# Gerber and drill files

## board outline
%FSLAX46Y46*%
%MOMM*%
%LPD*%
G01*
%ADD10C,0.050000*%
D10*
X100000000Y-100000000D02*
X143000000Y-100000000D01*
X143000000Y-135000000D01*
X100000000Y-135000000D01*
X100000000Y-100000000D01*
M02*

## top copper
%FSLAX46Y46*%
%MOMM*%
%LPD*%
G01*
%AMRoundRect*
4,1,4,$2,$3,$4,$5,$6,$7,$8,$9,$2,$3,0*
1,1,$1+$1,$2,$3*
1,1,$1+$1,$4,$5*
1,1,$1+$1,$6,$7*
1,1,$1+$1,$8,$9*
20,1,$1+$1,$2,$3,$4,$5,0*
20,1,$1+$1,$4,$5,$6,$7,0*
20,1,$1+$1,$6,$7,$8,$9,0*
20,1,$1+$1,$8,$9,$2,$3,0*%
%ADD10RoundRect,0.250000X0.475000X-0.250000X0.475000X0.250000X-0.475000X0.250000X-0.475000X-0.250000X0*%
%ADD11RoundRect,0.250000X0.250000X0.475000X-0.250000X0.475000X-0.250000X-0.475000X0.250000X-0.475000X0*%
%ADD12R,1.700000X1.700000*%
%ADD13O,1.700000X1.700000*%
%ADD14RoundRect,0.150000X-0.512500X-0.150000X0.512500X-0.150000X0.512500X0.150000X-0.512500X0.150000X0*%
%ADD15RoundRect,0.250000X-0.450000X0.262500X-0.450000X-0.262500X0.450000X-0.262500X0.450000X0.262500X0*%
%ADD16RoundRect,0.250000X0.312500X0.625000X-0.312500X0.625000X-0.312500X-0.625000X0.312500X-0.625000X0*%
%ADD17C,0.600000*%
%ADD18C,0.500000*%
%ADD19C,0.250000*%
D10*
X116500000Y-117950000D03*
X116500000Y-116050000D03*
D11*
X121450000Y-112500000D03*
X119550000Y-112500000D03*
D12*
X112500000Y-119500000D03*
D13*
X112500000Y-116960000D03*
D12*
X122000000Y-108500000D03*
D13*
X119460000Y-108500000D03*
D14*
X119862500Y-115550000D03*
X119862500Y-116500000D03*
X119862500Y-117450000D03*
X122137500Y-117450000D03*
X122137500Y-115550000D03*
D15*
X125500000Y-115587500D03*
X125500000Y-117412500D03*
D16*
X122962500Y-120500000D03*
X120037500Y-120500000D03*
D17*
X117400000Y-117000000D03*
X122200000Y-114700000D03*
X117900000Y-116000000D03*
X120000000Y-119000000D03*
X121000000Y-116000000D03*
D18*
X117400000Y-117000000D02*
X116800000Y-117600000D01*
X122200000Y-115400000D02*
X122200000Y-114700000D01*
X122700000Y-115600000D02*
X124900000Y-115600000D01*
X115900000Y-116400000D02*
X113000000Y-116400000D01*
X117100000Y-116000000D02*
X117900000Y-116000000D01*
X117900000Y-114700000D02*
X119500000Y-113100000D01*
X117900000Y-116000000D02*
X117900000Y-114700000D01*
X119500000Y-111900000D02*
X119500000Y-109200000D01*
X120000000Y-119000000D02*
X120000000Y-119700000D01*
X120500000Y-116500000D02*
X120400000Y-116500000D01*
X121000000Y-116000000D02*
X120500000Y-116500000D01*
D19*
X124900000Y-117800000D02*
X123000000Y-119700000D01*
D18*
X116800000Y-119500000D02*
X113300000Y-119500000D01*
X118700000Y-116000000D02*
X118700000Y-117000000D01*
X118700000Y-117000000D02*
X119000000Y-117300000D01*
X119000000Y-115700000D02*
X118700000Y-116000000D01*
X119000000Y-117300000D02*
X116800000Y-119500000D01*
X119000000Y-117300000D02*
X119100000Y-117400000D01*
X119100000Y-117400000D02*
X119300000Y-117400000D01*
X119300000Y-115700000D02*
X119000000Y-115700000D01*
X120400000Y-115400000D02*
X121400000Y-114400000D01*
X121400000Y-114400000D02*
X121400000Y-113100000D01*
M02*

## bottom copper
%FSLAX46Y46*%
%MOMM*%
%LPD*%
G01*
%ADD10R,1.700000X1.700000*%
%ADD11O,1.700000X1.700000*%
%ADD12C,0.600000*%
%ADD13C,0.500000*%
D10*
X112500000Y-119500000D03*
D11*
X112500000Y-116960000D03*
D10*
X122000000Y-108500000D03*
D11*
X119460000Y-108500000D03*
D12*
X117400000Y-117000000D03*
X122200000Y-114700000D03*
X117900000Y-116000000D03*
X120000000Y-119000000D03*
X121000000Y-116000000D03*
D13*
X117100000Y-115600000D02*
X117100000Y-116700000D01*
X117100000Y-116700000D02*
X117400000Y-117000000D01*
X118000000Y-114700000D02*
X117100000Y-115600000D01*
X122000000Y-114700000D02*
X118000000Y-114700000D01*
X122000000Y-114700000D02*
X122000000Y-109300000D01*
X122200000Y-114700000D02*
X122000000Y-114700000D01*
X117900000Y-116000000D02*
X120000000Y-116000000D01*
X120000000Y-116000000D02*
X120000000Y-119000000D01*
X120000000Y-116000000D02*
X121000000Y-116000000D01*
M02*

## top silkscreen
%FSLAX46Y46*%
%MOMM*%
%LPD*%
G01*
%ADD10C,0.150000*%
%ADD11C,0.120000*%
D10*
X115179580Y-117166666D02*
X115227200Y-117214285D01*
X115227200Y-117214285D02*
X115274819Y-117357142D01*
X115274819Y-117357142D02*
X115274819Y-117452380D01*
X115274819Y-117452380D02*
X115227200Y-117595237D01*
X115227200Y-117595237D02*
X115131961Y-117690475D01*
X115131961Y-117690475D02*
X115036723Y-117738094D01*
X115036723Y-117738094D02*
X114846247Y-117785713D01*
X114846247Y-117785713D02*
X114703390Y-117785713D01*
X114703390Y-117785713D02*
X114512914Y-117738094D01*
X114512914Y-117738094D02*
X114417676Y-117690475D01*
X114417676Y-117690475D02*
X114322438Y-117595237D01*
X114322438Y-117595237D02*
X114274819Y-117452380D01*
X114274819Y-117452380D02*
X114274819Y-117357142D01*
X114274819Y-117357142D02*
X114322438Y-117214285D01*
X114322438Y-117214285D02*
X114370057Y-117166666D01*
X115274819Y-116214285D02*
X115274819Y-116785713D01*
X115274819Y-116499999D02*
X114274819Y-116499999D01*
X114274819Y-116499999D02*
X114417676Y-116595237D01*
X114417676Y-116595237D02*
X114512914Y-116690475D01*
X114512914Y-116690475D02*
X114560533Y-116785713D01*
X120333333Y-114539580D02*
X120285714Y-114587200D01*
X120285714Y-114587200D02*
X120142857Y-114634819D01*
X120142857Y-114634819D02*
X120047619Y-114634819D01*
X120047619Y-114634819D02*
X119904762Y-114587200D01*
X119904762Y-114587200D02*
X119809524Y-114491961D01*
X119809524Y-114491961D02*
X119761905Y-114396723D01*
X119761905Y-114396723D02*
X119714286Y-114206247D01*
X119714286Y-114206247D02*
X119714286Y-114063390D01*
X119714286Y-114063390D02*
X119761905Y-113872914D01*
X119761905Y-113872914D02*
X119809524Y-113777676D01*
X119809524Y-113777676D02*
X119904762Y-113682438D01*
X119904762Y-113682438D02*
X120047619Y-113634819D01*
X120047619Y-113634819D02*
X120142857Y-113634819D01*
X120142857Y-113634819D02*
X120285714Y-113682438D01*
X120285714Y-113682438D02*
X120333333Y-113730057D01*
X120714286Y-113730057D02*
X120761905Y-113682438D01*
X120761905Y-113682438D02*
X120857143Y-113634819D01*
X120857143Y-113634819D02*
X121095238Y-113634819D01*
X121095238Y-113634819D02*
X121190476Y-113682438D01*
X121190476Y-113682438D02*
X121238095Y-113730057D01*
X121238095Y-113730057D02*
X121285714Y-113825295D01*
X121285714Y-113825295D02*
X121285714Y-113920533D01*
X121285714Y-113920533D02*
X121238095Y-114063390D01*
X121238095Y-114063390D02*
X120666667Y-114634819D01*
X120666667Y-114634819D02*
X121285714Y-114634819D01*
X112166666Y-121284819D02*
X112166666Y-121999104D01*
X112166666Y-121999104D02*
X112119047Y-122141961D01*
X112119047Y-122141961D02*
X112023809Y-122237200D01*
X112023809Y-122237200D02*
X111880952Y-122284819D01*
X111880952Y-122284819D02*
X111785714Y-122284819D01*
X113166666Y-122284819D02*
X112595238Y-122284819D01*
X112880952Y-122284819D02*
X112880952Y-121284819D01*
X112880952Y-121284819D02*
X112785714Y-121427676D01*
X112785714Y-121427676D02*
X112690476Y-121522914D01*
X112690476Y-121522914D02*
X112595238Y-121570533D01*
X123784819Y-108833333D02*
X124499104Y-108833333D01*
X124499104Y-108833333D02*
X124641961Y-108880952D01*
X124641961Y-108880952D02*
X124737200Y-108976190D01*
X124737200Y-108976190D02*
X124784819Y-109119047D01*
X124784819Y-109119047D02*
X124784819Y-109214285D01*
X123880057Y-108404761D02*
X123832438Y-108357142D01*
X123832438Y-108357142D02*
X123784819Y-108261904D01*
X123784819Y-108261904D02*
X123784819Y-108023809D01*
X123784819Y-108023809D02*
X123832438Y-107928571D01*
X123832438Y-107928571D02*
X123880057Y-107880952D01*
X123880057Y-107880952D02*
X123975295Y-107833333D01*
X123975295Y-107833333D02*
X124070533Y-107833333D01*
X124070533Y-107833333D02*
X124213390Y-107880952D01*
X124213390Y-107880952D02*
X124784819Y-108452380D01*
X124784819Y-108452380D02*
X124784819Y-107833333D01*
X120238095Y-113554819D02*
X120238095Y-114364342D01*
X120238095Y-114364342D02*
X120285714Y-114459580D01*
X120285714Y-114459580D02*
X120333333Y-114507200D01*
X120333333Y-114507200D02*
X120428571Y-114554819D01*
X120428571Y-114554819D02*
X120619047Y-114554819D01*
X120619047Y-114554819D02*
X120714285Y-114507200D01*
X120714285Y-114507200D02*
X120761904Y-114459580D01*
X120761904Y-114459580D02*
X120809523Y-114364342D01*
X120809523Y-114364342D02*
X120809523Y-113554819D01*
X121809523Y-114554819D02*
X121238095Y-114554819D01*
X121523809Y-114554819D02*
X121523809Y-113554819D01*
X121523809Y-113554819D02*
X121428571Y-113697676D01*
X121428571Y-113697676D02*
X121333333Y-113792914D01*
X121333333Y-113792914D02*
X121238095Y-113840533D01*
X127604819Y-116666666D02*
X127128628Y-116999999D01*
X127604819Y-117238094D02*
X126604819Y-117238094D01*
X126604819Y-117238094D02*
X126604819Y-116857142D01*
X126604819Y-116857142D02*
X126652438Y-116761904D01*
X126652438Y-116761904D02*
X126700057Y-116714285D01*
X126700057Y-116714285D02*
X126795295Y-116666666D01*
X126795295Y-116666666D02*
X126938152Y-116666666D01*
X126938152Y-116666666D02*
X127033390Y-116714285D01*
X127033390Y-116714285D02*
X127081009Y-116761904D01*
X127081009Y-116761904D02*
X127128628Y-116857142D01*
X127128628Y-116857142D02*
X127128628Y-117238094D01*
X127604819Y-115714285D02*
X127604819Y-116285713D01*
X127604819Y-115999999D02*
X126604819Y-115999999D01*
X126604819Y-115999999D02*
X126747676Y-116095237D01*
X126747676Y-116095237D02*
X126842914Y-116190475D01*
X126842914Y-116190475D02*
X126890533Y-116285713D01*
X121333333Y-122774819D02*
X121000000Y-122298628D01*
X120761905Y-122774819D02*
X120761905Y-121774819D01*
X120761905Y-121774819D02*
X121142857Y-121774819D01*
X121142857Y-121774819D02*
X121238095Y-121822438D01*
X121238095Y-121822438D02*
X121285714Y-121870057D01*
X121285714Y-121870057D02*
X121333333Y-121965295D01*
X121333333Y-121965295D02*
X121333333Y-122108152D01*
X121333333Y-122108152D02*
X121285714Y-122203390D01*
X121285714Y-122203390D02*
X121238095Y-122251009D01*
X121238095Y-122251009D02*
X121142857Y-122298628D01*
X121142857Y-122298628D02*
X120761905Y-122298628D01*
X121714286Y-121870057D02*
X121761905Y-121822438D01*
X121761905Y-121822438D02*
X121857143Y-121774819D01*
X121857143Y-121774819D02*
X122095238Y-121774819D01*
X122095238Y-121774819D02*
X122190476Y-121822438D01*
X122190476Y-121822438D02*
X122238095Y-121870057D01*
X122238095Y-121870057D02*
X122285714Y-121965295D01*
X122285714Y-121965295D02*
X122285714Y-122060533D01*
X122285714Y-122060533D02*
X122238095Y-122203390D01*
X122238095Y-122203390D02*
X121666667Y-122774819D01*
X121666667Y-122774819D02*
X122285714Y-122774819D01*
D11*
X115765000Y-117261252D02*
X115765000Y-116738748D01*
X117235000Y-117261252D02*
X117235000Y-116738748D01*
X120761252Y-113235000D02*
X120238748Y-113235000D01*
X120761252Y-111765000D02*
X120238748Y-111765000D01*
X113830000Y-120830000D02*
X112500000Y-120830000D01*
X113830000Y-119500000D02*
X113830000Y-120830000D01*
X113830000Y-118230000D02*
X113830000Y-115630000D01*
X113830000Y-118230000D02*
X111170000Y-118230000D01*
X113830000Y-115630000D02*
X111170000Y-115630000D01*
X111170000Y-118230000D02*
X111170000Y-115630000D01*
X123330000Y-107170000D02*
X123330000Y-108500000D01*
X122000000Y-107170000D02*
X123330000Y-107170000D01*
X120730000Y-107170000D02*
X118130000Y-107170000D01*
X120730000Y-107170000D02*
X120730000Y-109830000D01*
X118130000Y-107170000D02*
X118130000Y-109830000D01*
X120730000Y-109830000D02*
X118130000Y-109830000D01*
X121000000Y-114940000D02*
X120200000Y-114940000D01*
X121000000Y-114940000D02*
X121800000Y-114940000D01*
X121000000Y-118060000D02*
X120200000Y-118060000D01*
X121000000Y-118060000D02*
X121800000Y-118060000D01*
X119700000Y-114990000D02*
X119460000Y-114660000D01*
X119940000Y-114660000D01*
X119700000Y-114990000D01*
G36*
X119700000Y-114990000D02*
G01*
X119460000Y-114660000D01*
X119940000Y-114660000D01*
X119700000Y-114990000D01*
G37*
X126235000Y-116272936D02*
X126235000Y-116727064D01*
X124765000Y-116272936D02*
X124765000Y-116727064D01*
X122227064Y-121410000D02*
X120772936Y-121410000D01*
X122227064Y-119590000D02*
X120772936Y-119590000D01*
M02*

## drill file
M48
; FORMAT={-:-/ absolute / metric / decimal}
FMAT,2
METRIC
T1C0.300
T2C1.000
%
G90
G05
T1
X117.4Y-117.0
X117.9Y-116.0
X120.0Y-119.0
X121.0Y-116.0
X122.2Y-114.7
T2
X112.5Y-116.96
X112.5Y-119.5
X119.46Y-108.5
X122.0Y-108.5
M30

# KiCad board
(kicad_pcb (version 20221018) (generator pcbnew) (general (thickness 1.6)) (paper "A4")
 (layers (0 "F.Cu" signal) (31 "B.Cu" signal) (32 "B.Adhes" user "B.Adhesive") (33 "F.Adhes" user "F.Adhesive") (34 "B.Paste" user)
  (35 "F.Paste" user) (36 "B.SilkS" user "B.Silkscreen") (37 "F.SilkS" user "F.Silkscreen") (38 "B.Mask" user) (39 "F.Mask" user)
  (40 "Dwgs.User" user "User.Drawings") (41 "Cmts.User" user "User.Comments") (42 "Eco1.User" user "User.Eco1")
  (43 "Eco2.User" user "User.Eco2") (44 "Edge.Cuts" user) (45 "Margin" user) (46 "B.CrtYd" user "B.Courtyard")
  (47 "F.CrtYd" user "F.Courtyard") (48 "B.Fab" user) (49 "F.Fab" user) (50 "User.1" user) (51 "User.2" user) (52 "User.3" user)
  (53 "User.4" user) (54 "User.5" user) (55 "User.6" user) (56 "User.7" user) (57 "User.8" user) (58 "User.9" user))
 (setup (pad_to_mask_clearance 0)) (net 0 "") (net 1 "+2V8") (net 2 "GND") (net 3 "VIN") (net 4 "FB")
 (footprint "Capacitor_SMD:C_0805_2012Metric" (layer "F.Cu") (at 116.5 117 90)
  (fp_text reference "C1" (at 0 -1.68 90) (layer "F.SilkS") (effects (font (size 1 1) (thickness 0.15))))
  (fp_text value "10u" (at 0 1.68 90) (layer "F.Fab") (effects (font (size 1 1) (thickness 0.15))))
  (fp_line (start -0.261252 -0.735) (end 0.261252 -0.735) (stroke (width 0.12) (type solid)) (layer "F.SilkS"))
  (fp_line (start -0.261252 0.735) (end 0.261252 0.735) (stroke (width 0.12) (type solid)) (layer "F.SilkS"))
  (pad "1" smd roundrect (at -0.95 0 90) (size 1 1.45) (layers "F.Cu" "F.Paste" "F.Mask") (roundrect_rratio 0.25) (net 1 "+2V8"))
  (pad "2" smd roundrect (at 0.95 0 90) (size 1 1.45) (layers "F.Cu" "F.Paste" "F.Mask") (roundrect_rratio 0.25) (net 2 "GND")))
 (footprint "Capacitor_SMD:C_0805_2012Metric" (layer "F.Cu") (at 120.5 112.5 180)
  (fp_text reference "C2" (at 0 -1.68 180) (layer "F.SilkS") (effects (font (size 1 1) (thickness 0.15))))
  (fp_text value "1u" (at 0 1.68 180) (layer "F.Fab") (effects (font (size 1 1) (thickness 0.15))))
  (fp_line (start -0.261252 -0.735) (end 0.261252 -0.735) (stroke (width 0.12) (type solid)) (layer "F.SilkS"))
  (fp_line (start -0.261252 0.735) (end 0.261252 0.735) (stroke (width 0.12) (type solid)) (layer "F.SilkS"))
  (pad "1" smd roundrect (at -0.95 0 180) (size 1 1.45) (layers "F.Cu" "F.Paste" "F.Mask") (roundrect_rratio 0.25) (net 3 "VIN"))
  (pad "2" smd roundrect (at 0.95 0 180) (size 1 1.45) (layers "F.Cu" "F.Paste" "F.Mask") (roundrect_rratio 0.25) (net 2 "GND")))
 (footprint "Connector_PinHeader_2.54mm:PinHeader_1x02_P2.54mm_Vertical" (layer "F.Cu") (at 112.5 119.5 180)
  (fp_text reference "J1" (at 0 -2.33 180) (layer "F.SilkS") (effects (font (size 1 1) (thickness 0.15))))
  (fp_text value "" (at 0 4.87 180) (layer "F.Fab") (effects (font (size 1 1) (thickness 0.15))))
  (fp_line (start -1.33 -1.33) (end 0 -1.33) (stroke (width 0.12) (type solid)) (layer "F.SilkS"))
  (fp_line (start -1.33 0) (end -1.33 -1.33) (stroke (width 0.12) (type solid)) (layer "F.SilkS"))
  (fp_line (start -1.33 1.27) (end -1.33 3.87) (stroke (width 0.12) (type solid)) (layer "F.SilkS"))
  (fp_line (start -1.33 1.27) (end 1.33 1.27) (stroke (width 0.12) (type solid)) (layer "F.SilkS"))
  (fp_line (start -1.33 3.87) (end 1.33 3.87) (stroke (width 0.12) (type solid)) (layer "F.SilkS"))
  (fp_line (start 1.33 1.27) (end 1.33 3.87) (stroke (width 0.12) (type solid)) (layer "F.SilkS"))
  (pad "1" thru_hole rect (at 0 0 180) (size 1.7 1.7) (drill 1) (layers "*.Cu" "*.Mask") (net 3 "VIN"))
  (pad "2" thru_hole oval (at 0 2.54 180) (size 1.7 1.7) (drill 1) (layers "*.Cu" "*.Mask") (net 2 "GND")))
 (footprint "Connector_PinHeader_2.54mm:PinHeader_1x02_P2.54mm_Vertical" (layer "F.Cu") (at 122 108.5 -90)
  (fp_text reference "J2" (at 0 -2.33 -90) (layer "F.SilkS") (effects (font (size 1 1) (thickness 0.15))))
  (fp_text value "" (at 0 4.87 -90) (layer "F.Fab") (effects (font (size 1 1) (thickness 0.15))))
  (fp_line (start -1.33 -1.33) (end 0 -1.33) (stroke (width 0.12) (type solid)) (layer "F.SilkS"))
  (fp_line (start -1.33 0) (end -1.33 -1.33) (stroke (width 0.12) (type solid)) (layer "F.SilkS"))
  (fp_line (start -1.33 1.27) (end -1.33 3.87) (stroke (width 0.12) (type solid)) (layer "F.SilkS"))
  (fp_line (start -1.33 1.27) (end 1.33 1.27) (stroke (width 0.12) (type solid)) (layer "F.SilkS"))
  (fp_line (start -1.33 3.87) (end 1.33 3.87) (stroke (width 0.12) (type solid)) (layer "F.SilkS"))
  (fp_line (start 1.33 1.27) (end 1.33 3.87) (stroke (width 0.12) (type solid)) (layer "F.SilkS"))
  (pad "1" thru_hole rect (at 0 0 270) (size 1.7 1.7) (drill 1) (layers "*.Cu" "*.Mask") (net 1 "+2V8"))
  (pad "2" thru_hole oval (at 0 2.54 270) (size 1.7 1.7) (drill 1) (layers "*.Cu" "*.Mask") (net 2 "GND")))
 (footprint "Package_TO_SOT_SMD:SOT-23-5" (layer "F.Cu") (at 121 116.5)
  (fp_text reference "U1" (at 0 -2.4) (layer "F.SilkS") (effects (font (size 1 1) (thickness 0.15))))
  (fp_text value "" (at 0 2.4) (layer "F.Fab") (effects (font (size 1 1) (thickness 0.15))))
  (fp_line (start 0 -1.56) (end -0.8 -1.56) (stroke (width 0.12) (type solid)) (layer "F.SilkS"))
  (fp_line (start 0 -1.56) (end 0.8 -1.56) (stroke (width 0.12) (type solid)) (layer "F.SilkS"))
  (fp_line (start 0 1.56) (end -0.8 1.56) (stroke (width 0.12) (type solid)) (layer "F.SilkS"))
  (fp_line (start 0 1.56) (end 0.8 1.56) (stroke (width 0.12) (type solid)) (layer "F.SilkS"))
  (fp_poly
   (pts (xy -1.3 -1.51) (xy -1.54 -1.84) (xy -1.06 -1.84) (xy -1.3 -1.51)) (stroke (width 0.12) (type solid)) (fill solid) (layer "F.SilkS"))
  (pad "1" smd roundrect (at -1.1375 -0.95) (size 1.325 0.6) (layers "F.Cu" "F.Paste" "F.Mask") (roundrect_rratio 0.25) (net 3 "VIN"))
  (pad "2" smd roundrect (at -1.1375 0) (size 1.325 0.6) (layers "F.Cu" "F.Paste" "F.Mask") (roundrect_rratio 0.25) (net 2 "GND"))
  (pad "3" smd roundrect (at -1.1375 0.95) (size 1.325 0.6) (layers "F.Cu" "F.Paste" "F.Mask") (roundrect_rratio 0.25) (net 3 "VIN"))
  (pad "4" smd roundrect (at 1.1375 0.95) (size 1.325 0.6) (layers "F.Cu" "F.Paste" "F.Mask") (roundrect_rratio 0.25))
  (pad "5" smd roundrect (at 1.1375 -0.95) (size 1.325 0.6) (layers "F.Cu" "F.Paste" "F.Mask") (roundrect_rratio 0.25) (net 1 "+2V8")))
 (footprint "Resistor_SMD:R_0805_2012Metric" (layer "F.Cu") (at 125.5 116.5 -90)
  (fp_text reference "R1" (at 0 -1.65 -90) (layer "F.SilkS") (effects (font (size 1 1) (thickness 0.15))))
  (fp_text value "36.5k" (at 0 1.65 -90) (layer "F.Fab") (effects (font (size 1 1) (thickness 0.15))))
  (fp_line (start -0.227064 -0.735) (end 0.227064 -0.735) (stroke (width 0.12) (type solid)) (layer "F.SilkS"))
  (fp_line (start -0.227064 0.735) (end 0.227064 0.735) (stroke (width 0.12) (type solid)) (layer "F.SilkS"))
  (pad "1" smd roundrect (at -0.9125 0 270) (size 1.025 1.4) (layers "F.Cu" "F.Paste" "F.Mask") (roundrect_rratio 0.243902) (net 1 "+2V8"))
  (pad "2" smd roundrect (at 0.9125 0 270) (size 1.025 1.4) (layers "F.Cu" "F.Paste" "F.Mask") (roundrect_rratio 0.243902) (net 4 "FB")))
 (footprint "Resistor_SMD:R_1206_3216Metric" (layer "F.Cu") (at 121.5 120.5 180)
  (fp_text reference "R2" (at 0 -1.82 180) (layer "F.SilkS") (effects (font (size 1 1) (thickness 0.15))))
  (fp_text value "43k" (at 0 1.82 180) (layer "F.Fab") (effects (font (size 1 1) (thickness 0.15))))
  (fp_line (start -0.727064 -0.91) (end 0.727064 -0.91) (stroke (width 0.12) (type solid)) (layer "F.SilkS"))
  (fp_line (start -0.727064 0.91) (end 0.727064 0.91) (stroke (width 0.12) (type solid)) (layer "F.SilkS"))
  (pad "1" smd roundrect (at -1.4625 0 180) (size 1.125 1.75) (layers "F.Cu" "F.Paste" "F.Mask") (roundrect_rratio 0.222222) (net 4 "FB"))
  (pad "2" smd roundrect (at 1.4625 0 180) (size 1.125 1.75) (layers "F.Cu" "F.Paste" "F.Mask") (roundrect_rratio 0.222222) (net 2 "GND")))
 (gr_rect (start 100 100) (end 143 135) (stroke (width 0.05) (type default)) (fill none) (layer "Edge.Cuts"))
 (segment (start 117.4 117) (end 116.8 117.6) (width 0.5) (layer "F.Cu") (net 1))
 (segment (start 122.2 115.4) (end 122.2 114.7) (width 0.5) (layer "F.Cu") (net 1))
 (segment (start 122.7 115.6) (end 124.9 115.6) (width 0.5) (layer "F.Cu") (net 1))
 (via (at 117.4 117) (size 0.6) (drill 0.3) (layers "F.Cu" "B.Cu") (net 1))
 (via (at 122.2 114.7) (size 0.6) (drill 0.3) (layers "F.Cu" "B.Cu") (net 1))
 (segment (start 115.9 116.4) (end 113 116.4) (width 0.5) (layer "F.Cu") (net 2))
 (segment (start 117.1 115.6) (end 117.1 116.7) (width 0.5) (layer "B.Cu") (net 1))
 (segment (start 117.1 116) (end 117.9 116) (width 0.5) (layer "F.Cu") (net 2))
 (segment (start 117.1 116.7) (end 117.4 117) (width 0.5) (layer "B.Cu") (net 1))
 (segment (start 117.9 114.7) (end 119.5 113.1) (width 0.5) (layer "F.Cu") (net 2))
 (segment (start 117.9 116) (end 117.9 114.7) (width 0.5) (layer "F.Cu") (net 2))
 (segment (start 118 114.7) (end 117.1 115.6) (width 0.5) (layer "B.Cu") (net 1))
 (segment (start 119.5 111.9) (end 119.5 109.2) (width 0.5) (layer "F.Cu") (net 2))
 (segment (start 120 119) (end 120 119.7) (width 0.5) (layer "F.Cu") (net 2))
 (segment (start 120.5 116.5) (end 120.4 116.5) (width 0.5) (layer "F.Cu") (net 2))
 (segment (start 121 116) (end 120.5 116.5) (width 0.5) (layer "F.Cu") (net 2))
 (segment (start 122 114.7) (end 118 114.7) (width 0.5) (layer "B.Cu") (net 1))
 (segment (start 122 114.7) (end 122 109.3) (width 0.5) (layer "B.Cu") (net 1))
 (segment (start 122.2 114.7) (end 122 114.7) (width 0.5) (layer "B.Cu") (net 1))
 (segment (start 124.9 117.8) (end 123 119.7) (width 0.25) (layer "F.Cu") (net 4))
 (via (at 117.9 116) (size 0.6) (drill 0.3) (layers "F.Cu" "B.Cu") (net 2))
 (via (at 120 119) (size 0.6) (drill 0.3) (layers "F.Cu" "B.Cu") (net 2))
 (via (at 121 116) (size 0.6) (drill 0.3) (layers "F.Cu" "B.Cu") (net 2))
 (segment (start 116.8 119.5) (end 113.3 119.5) (width 0.5) (layer "F.Cu") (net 3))
 (segment (start 117.9 116) (end 120 116) (width 0.5) (layer "B.Cu") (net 2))
 (segment (start 118.7 116) (end 118.7 117) (width 0.5) (layer "F.Cu") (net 3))
 (segment (start 118.7 117) (end 119 117.3) (width 0.5) (layer "F.Cu") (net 3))
 (segment (start 119 115.7) (end 118.7 116) (width 0.5) (layer "F.Cu") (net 3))
 (segment (start 119 117.3) (end 116.8 119.5) (width 0.5) (layer "F.Cu") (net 3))
 (segment (start 119 117.3) (end 119.1 117.4) (width 0.5) (layer "F.Cu") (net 3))
 (segment (start 119.1 117.4) (end 119.3 117.4) (width 0.5) (layer "F.Cu") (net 3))
 (segment (start 119.3 115.7) (end 119 115.7) (width 0.5) (layer "F.Cu") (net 3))
 (segment (start 120 116) (end 120 119) (width 0.5) (layer "B.Cu") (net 2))
 (segment (start 120 116) (end 121 116) (width 0.5) (layer "B.Cu") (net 2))
 (segment (start 120.4 115.4) (end 121.4 114.4) (width 0.5) (layer "F.Cu") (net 3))
 (segment (start 121.4 114.4) (end 121.4 113.1) (width 0.5) (layer "F.Cu") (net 3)))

